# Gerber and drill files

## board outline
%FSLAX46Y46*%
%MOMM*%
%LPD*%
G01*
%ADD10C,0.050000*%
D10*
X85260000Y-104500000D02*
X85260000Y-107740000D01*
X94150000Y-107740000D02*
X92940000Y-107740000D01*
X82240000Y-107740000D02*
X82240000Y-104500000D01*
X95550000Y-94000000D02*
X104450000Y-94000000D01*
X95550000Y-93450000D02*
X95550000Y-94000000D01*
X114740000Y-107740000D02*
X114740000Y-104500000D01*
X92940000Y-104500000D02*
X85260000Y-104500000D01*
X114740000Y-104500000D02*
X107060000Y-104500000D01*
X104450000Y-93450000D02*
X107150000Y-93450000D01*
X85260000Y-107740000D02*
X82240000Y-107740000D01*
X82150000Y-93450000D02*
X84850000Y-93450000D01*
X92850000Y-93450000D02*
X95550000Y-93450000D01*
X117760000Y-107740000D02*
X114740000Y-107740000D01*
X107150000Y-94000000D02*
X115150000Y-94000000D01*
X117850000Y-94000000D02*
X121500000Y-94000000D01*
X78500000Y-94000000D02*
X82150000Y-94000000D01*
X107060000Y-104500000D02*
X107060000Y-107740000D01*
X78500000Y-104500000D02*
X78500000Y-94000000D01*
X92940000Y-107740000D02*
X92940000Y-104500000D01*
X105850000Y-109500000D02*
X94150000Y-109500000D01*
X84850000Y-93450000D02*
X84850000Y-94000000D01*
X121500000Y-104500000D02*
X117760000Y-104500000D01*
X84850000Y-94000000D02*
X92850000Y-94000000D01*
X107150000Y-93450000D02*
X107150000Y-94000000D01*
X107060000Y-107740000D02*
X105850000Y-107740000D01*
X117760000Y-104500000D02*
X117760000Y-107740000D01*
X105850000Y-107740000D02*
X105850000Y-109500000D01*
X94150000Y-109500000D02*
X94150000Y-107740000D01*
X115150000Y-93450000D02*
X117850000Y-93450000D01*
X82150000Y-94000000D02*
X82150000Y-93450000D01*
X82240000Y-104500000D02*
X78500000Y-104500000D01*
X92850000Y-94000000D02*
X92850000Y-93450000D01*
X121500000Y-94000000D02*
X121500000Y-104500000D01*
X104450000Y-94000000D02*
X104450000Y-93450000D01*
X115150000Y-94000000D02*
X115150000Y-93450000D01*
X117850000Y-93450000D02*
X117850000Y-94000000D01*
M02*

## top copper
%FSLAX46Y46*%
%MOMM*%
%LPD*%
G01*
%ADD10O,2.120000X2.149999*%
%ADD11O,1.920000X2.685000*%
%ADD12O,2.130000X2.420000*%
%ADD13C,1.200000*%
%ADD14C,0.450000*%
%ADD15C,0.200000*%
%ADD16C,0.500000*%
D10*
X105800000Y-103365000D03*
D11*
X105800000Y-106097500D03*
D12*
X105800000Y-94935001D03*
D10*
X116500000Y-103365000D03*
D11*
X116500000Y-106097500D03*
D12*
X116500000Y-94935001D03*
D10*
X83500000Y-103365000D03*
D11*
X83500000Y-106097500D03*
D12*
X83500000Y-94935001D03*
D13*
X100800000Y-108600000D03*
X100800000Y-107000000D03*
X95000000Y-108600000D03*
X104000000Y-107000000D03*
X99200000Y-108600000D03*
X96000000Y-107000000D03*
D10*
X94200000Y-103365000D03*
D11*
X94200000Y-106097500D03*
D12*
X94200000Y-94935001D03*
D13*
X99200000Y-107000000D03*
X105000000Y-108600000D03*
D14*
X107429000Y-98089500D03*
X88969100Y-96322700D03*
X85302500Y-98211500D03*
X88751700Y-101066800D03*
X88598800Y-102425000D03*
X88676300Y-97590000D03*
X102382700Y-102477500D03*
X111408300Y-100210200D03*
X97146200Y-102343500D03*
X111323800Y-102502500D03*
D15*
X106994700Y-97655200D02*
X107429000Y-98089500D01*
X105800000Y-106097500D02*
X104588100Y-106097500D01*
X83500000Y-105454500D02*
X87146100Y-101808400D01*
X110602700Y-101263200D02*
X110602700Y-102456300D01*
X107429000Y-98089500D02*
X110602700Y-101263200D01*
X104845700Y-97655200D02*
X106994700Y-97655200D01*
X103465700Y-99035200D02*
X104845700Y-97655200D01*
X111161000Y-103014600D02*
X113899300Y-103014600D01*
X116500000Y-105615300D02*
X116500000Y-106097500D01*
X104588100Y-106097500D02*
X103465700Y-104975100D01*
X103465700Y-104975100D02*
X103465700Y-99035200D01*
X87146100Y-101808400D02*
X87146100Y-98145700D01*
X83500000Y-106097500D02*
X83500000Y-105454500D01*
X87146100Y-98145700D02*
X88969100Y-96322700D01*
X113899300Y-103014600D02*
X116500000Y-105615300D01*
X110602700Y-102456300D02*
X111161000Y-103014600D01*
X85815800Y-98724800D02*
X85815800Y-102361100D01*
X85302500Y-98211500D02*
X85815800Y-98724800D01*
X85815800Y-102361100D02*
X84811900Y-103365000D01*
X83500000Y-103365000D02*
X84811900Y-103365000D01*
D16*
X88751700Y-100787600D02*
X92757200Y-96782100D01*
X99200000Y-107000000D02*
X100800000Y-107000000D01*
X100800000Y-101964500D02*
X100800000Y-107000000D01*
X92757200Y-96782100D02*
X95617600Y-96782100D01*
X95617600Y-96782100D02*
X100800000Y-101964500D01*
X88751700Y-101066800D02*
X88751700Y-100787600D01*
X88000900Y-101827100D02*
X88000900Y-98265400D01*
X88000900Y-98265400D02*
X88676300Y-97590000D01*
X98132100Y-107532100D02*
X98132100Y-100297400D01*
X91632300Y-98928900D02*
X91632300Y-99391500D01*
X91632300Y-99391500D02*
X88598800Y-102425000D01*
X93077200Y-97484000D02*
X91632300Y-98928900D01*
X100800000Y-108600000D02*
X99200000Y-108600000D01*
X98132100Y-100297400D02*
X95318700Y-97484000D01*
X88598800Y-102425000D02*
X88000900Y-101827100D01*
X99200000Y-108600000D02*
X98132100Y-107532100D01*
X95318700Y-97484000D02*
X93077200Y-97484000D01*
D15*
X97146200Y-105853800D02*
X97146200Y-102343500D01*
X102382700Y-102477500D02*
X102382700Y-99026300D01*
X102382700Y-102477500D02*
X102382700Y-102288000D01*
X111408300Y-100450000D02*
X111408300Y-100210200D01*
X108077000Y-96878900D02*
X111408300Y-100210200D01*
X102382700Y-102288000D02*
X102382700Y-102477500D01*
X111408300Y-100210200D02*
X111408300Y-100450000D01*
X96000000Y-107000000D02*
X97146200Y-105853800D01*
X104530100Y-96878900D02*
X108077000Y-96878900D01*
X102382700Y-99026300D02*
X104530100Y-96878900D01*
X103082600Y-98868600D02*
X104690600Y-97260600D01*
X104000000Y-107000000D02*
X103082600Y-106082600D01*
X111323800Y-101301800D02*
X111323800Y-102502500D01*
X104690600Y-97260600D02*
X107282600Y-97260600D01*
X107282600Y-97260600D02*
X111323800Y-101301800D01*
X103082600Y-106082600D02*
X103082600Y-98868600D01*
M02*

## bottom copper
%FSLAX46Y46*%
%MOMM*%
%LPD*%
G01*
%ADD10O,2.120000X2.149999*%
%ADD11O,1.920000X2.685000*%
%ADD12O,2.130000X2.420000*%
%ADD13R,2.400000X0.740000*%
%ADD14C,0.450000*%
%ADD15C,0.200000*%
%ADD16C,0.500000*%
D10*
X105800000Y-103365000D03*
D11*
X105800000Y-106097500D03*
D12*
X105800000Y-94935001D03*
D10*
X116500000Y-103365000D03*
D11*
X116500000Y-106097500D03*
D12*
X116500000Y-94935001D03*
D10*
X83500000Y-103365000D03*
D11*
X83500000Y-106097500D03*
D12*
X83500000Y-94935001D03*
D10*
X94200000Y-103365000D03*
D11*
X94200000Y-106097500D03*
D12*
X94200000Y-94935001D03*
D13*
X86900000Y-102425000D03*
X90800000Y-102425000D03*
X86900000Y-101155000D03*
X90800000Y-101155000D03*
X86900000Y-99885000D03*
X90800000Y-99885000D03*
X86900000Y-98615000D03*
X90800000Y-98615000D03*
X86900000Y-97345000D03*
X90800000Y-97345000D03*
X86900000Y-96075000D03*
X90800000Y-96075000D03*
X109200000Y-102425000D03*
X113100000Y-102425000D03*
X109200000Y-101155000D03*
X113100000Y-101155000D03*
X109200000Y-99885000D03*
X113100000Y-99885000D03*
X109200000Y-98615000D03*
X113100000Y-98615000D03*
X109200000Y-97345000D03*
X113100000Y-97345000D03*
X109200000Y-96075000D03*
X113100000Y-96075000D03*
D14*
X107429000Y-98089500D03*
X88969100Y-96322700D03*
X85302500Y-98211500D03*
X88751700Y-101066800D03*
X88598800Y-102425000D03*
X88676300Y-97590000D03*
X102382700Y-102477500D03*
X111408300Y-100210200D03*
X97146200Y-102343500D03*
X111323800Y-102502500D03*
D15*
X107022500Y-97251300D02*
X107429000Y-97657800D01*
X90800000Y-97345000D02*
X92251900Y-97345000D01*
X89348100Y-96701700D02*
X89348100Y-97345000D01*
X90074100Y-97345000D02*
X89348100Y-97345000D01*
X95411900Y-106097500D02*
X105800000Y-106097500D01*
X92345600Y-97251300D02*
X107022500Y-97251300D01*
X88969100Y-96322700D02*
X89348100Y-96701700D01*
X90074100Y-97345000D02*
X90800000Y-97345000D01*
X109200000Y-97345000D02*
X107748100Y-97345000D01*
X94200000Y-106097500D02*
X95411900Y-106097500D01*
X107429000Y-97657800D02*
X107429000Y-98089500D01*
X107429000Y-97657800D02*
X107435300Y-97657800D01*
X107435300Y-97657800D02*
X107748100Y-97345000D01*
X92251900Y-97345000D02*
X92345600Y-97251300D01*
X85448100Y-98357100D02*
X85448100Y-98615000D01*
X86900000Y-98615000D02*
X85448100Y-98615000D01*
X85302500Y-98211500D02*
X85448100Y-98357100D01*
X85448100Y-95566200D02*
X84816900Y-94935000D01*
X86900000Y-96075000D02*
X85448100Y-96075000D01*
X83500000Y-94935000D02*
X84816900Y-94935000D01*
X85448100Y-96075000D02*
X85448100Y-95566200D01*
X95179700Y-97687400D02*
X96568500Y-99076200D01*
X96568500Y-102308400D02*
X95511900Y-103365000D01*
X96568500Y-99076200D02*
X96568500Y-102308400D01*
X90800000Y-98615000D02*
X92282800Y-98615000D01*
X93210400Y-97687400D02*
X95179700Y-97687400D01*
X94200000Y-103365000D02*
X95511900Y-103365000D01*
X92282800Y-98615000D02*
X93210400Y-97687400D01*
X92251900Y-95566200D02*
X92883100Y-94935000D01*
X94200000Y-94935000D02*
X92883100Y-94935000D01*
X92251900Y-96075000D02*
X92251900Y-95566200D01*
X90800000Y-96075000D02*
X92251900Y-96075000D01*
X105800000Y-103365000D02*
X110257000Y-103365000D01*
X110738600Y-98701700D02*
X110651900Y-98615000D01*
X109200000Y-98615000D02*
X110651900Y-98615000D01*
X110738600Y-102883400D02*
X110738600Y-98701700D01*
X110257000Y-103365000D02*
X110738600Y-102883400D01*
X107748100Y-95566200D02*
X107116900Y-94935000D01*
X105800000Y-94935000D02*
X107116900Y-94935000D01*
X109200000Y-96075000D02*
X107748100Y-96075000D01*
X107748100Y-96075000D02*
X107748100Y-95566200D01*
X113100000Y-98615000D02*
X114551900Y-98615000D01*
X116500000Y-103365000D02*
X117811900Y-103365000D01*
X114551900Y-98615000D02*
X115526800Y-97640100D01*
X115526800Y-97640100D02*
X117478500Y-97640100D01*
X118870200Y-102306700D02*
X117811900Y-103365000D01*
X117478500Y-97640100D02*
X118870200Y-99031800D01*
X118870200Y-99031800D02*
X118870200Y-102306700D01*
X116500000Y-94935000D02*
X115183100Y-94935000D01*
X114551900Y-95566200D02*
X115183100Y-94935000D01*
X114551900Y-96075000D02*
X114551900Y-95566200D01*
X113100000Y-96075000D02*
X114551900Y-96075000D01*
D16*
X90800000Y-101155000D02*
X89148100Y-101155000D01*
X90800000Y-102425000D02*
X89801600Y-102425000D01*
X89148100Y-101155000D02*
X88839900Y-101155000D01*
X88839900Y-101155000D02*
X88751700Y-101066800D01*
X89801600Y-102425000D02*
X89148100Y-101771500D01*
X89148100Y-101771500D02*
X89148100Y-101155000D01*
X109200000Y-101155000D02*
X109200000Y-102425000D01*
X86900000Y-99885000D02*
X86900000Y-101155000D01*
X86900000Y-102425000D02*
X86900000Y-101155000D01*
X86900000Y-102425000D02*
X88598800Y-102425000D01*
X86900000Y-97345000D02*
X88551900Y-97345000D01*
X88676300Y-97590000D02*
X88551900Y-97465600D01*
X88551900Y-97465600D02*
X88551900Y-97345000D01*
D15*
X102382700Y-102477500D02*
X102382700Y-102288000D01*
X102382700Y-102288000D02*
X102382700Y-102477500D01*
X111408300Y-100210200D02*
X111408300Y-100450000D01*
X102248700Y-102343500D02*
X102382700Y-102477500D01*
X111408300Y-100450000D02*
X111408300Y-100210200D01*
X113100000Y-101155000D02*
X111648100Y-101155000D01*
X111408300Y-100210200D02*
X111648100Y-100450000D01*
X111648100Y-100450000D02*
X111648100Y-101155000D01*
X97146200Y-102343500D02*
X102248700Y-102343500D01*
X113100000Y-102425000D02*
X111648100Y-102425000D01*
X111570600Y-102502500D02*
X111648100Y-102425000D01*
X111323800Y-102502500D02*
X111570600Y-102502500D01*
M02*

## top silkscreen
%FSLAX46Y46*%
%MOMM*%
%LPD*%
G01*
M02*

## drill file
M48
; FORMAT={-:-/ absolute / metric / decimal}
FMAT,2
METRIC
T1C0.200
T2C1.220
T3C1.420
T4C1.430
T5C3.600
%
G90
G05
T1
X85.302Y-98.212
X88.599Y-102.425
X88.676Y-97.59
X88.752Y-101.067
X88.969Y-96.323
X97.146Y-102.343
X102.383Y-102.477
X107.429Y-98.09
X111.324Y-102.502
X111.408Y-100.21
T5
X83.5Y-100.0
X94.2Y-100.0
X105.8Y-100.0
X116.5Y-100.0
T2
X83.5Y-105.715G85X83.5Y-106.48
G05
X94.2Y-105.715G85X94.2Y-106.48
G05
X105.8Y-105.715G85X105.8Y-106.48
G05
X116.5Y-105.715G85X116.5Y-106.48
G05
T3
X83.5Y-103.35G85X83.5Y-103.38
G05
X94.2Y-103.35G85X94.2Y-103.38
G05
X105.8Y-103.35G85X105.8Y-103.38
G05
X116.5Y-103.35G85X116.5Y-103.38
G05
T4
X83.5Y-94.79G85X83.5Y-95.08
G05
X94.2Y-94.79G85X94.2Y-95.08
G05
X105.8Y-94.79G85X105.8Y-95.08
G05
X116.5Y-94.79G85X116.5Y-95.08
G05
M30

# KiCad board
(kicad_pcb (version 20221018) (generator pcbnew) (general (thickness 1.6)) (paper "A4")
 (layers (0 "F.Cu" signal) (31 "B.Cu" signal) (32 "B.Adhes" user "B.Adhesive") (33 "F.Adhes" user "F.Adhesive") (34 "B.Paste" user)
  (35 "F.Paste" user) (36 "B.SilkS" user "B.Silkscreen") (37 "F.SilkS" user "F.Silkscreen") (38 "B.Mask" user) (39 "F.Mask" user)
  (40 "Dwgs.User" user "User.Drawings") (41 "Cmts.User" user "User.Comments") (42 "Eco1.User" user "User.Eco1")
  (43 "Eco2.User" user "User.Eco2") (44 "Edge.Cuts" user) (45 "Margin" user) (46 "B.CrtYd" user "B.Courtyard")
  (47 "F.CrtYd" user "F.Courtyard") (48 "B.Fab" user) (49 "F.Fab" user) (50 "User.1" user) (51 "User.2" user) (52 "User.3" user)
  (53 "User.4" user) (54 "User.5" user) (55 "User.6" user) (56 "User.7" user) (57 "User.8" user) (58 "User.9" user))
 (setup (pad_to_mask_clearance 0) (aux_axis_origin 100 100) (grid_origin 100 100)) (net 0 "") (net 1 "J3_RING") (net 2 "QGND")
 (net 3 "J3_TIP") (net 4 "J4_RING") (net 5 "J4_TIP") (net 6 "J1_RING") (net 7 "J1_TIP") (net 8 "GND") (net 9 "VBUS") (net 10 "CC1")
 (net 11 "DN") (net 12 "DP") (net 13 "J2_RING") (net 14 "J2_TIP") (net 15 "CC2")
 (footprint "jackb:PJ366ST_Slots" (layer "F.Cu") (at 105.8 100)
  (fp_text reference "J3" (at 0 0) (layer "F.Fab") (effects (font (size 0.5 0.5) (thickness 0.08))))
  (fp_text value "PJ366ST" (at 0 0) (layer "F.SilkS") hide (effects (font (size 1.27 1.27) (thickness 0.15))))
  (pad "" np_thru_hole circle (at 0 0) (size 3.6 3.6) (drill 3.6) (layers "F&B.Cu" "*.Mask"))
  (pad "R" thru_hole oval (at 0 3.365) (size 2.12 2.149999) (drill oval 1.42 1.449999) (layers "*.Cu" "*.Mask") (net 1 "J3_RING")
   (thermal_bridge_angle 45))
  (pad "S" thru_hole oval (at 0 6.0975) (size 1.92 2.685) (drill oval 1.22 1.985) (layers "*.Cu" "*.Mask") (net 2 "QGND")
   (thermal_bridge_angle 45))
  (pad "T" thru_hole oval (at 0 -5.064999) (size 2.13 2.42) (drill oval 1.43 1.72) (layers "*.Cu" "*.Mask") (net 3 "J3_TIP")
   (thermal_bridge_angle 45)))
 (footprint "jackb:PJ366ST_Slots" (layer "F.Cu") (at 116.5 100)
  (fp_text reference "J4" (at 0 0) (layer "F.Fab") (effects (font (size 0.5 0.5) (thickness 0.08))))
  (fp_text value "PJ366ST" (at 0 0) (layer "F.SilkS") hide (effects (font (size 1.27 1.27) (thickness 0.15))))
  (pad "" np_thru_hole circle (at 0 0) (size 3.6 3.6) (drill 3.6) (layers "F&B.Cu" "*.Mask"))
  (pad "R" thru_hole oval (at 0 3.365) (size 2.12 2.149999) (drill oval 1.42 1.449999) (layers "*.Cu" "*.Mask") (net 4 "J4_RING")
   (thermal_bridge_angle 45))
  (pad "S" thru_hole oval (at 0 6.0975) (size 1.92 2.685) (drill oval 1.22 1.985) (layers "*.Cu" "*.Mask") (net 2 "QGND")
   (thermal_bridge_angle 45))
  (pad "T" thru_hole oval (at 0 -5.064999) (size 2.13 2.42) (drill oval 1.43 1.72) (layers "*.Cu" "*.Mask") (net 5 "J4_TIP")
   (thermal_bridge_angle 45)))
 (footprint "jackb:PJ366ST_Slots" (layer "F.Cu") (at 83.5 100)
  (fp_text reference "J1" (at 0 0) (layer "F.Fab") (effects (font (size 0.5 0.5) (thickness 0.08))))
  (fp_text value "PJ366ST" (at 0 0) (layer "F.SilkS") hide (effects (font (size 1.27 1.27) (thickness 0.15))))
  (pad "" np_thru_hole circle (at 0 0) (size 3.6 3.6) (drill 3.6) (layers "F&B.Cu" "*.Mask"))
  (pad "R" thru_hole oval (at 0 3.365) (size 2.12 2.149999) (drill oval 1.42 1.449999) (layers "*.Cu" "*.Mask") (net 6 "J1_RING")
   (thermal_bridge_angle 45))
  (pad "S" thru_hole oval (at 0 6.0975) (size 1.92 2.685) (drill oval 1.22 1.985) (layers "*.Cu" "*.Mask") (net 2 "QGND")
   (thermal_bridge_angle 45))
  (pad "T" thru_hole oval (at 0 -5.064999) (size 2.13 2.42) (drill oval 1.43 1.72) (layers "*.Cu" "*.Mask") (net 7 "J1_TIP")
   (thermal_bridge_angle 45)))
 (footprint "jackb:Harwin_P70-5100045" (layer "F.Cu") (at 100.8 108.6)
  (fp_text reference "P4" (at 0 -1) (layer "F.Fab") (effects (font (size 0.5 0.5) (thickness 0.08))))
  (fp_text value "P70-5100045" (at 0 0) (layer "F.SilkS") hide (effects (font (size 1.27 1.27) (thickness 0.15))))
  (pad "1" smd circle (at 0 0) (size 1.2 1.2) (layers "F.Cu" "F.Paste" "F.Mask") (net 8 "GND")))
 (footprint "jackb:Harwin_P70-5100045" (layer "F.Cu") (at 100.8 107)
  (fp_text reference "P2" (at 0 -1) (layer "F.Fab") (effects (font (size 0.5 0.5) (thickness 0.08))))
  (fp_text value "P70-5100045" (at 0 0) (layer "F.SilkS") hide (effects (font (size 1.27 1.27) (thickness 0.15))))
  (pad "1" smd circle (at 0 0) (size 1.2 1.2) (layers "F.Cu" "F.Paste" "F.Mask") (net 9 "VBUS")))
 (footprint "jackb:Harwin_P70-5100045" (layer "F.Cu") (at 95 108.6)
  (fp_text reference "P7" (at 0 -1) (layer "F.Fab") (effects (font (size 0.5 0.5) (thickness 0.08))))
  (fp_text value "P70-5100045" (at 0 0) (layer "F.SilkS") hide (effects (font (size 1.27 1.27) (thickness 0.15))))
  (pad "1" smd circle (at 0 0) (size 1.2 1.2) (layers "F.Cu" "F.Paste" "F.Mask") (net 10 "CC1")))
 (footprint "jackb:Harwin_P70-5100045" (layer "F.Cu") (at 104 107)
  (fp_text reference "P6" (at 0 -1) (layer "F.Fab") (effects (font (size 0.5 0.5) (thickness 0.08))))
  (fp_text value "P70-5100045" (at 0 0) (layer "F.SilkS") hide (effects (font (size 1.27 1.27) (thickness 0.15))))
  (pad "1" smd circle (at 0 0) (size 1.2 1.2) (layers "F.Cu" "F.Paste" "F.Mask") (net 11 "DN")))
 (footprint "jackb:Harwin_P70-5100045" (layer "F.Cu") (at 99.2 108.6)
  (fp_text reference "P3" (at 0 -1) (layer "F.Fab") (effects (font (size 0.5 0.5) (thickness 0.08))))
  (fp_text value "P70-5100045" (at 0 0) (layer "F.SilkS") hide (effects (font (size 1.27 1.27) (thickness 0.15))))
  (pad "1" smd circle (at 0 0) (size 1.2 1.2) (layers "F.Cu" "F.Paste" "F.Mask") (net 8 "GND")))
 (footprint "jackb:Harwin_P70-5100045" (layer "F.Cu") (at 96 107)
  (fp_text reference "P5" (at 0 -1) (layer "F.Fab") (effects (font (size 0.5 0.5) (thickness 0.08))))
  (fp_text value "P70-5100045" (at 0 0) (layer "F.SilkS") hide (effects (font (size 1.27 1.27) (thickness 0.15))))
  (pad "1" smd circle (at 0 0) (size 1.2 1.2) (layers "F.Cu" "F.Paste" "F.Mask") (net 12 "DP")))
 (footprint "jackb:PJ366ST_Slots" (layer "F.Cu") (at 94.2 100)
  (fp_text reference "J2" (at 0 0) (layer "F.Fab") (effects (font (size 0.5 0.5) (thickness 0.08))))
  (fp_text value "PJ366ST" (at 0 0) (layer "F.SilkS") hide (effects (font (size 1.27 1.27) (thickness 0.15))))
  (pad "" np_thru_hole circle (at 0 0) (size 3.6 3.6) (drill 3.6) (layers "F&B.Cu" "*.Mask"))
  (pad "R" thru_hole oval (at 0 3.365) (size 2.12 2.149999) (drill oval 1.42 1.449999) (layers "*.Cu" "*.Mask") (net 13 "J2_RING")
   (thermal_bridge_angle 45))
  (pad "S" thru_hole oval (at 0 6.0975) (size 1.92 2.685) (drill oval 1.22 1.985) (layers "*.Cu" "*.Mask") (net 2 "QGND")
   (thermal_bridge_angle 45))
  (pad "T" thru_hole oval (at 0 -5.064999) (size 2.13 2.42) (drill oval 1.43 1.72) (layers "*.Cu" "*.Mask") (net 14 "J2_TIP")
   (thermal_bridge_angle 45)))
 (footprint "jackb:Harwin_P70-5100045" (layer "F.Cu") (at 99.2 107)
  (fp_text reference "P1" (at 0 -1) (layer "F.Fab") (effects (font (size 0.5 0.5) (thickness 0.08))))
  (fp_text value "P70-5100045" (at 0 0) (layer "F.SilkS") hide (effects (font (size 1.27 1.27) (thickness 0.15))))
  (pad "1" smd circle (at 0 0) (size 1.2 1.2) (layers "F.Cu" "F.Paste" "F.Mask") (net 9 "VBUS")))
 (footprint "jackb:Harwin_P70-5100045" (layer "F.Cu") (at 105 108.6)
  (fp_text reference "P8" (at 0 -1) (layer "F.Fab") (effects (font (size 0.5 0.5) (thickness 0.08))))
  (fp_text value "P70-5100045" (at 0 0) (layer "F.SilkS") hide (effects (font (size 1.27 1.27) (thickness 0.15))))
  (pad "1" smd circle (at 0 0) (size 1.2 1.2) (layers "F.Cu" "F.Paste" "F.Mask") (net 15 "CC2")))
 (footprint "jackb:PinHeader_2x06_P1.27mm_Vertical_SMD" (layer "B.Cu") (at 88.85 99.25)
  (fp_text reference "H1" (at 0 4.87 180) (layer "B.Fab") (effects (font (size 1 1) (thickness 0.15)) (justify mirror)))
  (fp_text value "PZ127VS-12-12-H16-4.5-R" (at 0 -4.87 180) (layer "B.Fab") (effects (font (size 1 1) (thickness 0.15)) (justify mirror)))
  (pad "1" smd rect (at -1.95 3.175) (size 2.4 0.74) (layers "B.Cu" "B.Paste" "B.Mask") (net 8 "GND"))
  (pad "2" smd rect (at 1.95 3.175) (size 2.4 0.74) (layers "B.Cu" "B.Paste" "B.Mask") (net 9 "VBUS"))
  (pad "3" smd rect (at -1.95 1.905) (size 2.4 0.74) (layers "B.Cu" "B.Paste" "B.Mask") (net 8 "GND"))
  (pad "4" smd rect (at 1.95 1.905) (size 2.4 0.74) (layers "B.Cu" "B.Paste" "B.Mask") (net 9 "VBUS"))
  (pad "5" smd rect (at -1.95 0.635) (size 2.4 0.74) (layers "B.Cu" "B.Paste" "B.Mask") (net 8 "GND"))
  (pad "6" smd rect (at 1.95 0.635) (size 2.4 0.74) (layers "B.Cu" "B.Paste" "B.Mask") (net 10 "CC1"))
  (pad "7" smd rect (at -1.95 -0.635) (size 2.4 0.74) (layers "B.Cu" "B.Paste" "B.Mask") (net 6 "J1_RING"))
  (pad "8" smd rect (at 1.95 -0.635) (size 2.4 0.74) (layers "B.Cu" "B.Paste" "B.Mask") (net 13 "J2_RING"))
  (pad "9" smd rect (at -1.95 -1.905) (size 2.4 0.74) (layers "B.Cu" "B.Paste" "B.Mask") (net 8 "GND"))
  (pad "10" smd rect (at 1.95 -1.905) (size 2.4 0.74) (layers "B.Cu" "B.Paste" "B.Mask") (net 2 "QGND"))
  (pad "11" smd rect (at -1.95 -3.175) (size 2.4 0.74) (layers "B.Cu" "B.Paste" "B.Mask") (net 7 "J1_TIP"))
  (pad "12" smd rect (at 1.95 -3.175) (size 2.4 0.74) (layers "B.Cu" "B.Paste" "B.Mask") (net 14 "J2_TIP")))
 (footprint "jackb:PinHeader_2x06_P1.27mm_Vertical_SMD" (layer "B.Cu") (at 111.15 99.25)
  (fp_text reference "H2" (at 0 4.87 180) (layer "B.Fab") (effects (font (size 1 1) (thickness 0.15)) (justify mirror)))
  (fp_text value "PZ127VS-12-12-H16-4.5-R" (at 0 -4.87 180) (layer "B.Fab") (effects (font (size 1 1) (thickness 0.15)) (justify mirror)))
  (pad "1" smd rect (at -1.95 3.175) (size 2.4 0.74) (layers "B.Cu" "B.Paste" "B.Mask") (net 9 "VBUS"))
  (pad "2" smd rect (at 1.95 3.175) (size 2.4 0.74) (layers "B.Cu" "B.Paste" "B.Mask") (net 11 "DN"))
  (pad "3" smd rect (at -1.95 1.905) (size 2.4 0.74) (layers "B.Cu" "B.Paste" "B.Mask") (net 9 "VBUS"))
  (pad "4" smd rect (at 1.95 1.905) (size 2.4 0.74) (layers "B.Cu" "B.Paste" "B.Mask") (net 12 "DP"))
  (pad "5" smd rect (at -1.95 0.635) (size 2.4 0.74) (layers "B.Cu" "B.Paste" "B.Mask") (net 15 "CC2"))
  (pad "6" smd rect (at 1.95 0.635) (size 2.4 0.74) (layers "B.Cu" "B.Paste" "B.Mask") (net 8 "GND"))
  (pad "7" smd rect (at -1.95 -0.635) (size 2.4 0.74) (layers "B.Cu" "B.Paste" "B.Mask") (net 1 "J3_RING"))
  (pad "8" smd rect (at 1.95 -0.635) (size 2.4 0.74) (layers "B.Cu" "B.Paste" "B.Mask") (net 4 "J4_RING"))
  (pad "9" smd rect (at -1.95 -1.905) (size 2.4 0.74) (layers "B.Cu" "B.Paste" "B.Mask") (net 2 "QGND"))
  (pad "10" smd rect (at 1.95 -1.905) (size 2.4 0.74) (layers "B.Cu" "B.Paste" "B.Mask") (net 8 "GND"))
  (pad "11" smd rect (at -1.95 -3.175) (size 2.4 0.74) (layers "B.Cu" "B.Paste" "B.Mask") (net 3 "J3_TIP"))
  (pad "12" smd rect (at 1.95 -3.175) (size 2.4 0.74) (layers "B.Cu" "B.Paste" "B.Mask") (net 5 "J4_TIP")))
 (gr_line (start 85.26 104.5) (end 85.26 107.74) (stroke (width 0.05) (type default)) (layer "Edge.Cuts"))
 (gr_line (start 94.15 107.74) (end 92.94 107.74) (stroke (width 0.05) (type default)) (layer "Edge.Cuts"))
 (gr_line (start 82.24 107.74) (end 82.24 104.5) (stroke (width 0.05) (type default)) (layer "Edge.Cuts"))
 (gr_line (start 95.55 94) (end 104.45 94) (stroke (width 0.05) (type default)) (layer "Edge.Cuts"))
 (gr_line (start 95.55 93.45) (end 95.55 94) (stroke (width 0.05) (type default)) (layer "Edge.Cuts"))
 (gr_line (start 114.74 107.74) (end 114.74 104.5) (stroke (width 0.05) (type default)) (layer "Edge.Cuts"))
 (gr_line (start 92.94 104.5) (end 85.26 104.5) (stroke (width 0.05) (type default)) (layer "Edge.Cuts"))
 (gr_line (start 114.74 104.5) (end 107.06 104.5) (stroke (width 0.05) (type default)) (layer "Edge.Cuts"))
 (gr_line (start 104.45 93.45) (end 107.15 93.45) (stroke (width 0.05) (type default)) (layer "Edge.Cuts"))
 (gr_line (start 85.26 107.74) (end 82.24 107.74) (stroke (width 0.05) (type default)) (layer "Edge.Cuts"))
 (gr_line (start 82.15 93.45) (end 84.85 93.45) (stroke (width 0.05) (type default)) (layer "Edge.Cuts"))
 (gr_line (start 92.85 93.45) (end 95.55 93.45) (stroke (width 0.05) (type default)) (layer "Edge.Cuts"))
 (gr_line (start 117.76 107.74) (end 114.74 107.74) (stroke (width 0.05) (type default)) (layer "Edge.Cuts"))
 (gr_line (start 107.15 94) (end 115.15 94) (stroke (width 0.05) (type default)) (layer "Edge.Cuts"))
 (gr_line (start 117.85 94) (end 121.5 94) (stroke (width 0.05) (type default)) (layer "Edge.Cuts"))
 (gr_line (start 78.5 94) (end 82.15 94) (stroke (width 0.05) (type default)) (layer "Edge.Cuts"))
 (gr_line (start 107.06 104.5) (end 107.06 107.74) (stroke (width 0.05) (type default)) (layer "Edge.Cuts"))
 (gr_line (start 78.5 104.5) (end 78.5 94) (stroke (width 0.05) (type default)) (layer "Edge.Cuts"))
 (gr_line (start 92.94 107.74) (end 92.94 104.5) (stroke (width 0.05) (type default)) (layer "Edge.Cuts"))
 (gr_line (start 105.85 109.5) (end 94.15 109.5) (stroke (width 0.05) (type default)) (layer "Edge.Cuts"))
 (gr_line (start 84.85 93.45) (end 84.85 94) (stroke (width 0.05) (type default)) (layer "Edge.Cuts"))
 (gr_line (start 121.5 104.5) (end 117.76 104.5) (stroke (width 0.05) (type default)) (layer "Edge.Cuts"))
 (gr_line (start 84.85 94) (end 92.85 94) (stroke (width 0.05) (type default)) (layer "Edge.Cuts"))
 (gr_line (start 107.15 93.45) (end 107.15 94) (stroke (width 0.05) (type default)) (layer "Edge.Cuts"))
 (gr_line (start 107.06 107.74) (end 105.85 107.74) (stroke (width 0.05) (type default)) (layer "Edge.Cuts"))
 (gr_line (start 117.76 104.5) (end 117.76 107.74) (stroke (width 0.05) (type default)) (layer "Edge.Cuts"))
 (gr_line (start 105.85 107.74) (end 105.85 109.5) (stroke (width 0.05) (type default)) (layer "Edge.Cuts"))
 (gr_line (start 94.15 109.5) (end 94.15 107.74) (stroke (width 0.05) (type default)) (layer "Edge.Cuts"))
 (gr_line (start 115.15 93.45) (end 117.85 93.45) (stroke (width 0.05) (type default)) (layer "Edge.Cuts"))
 (gr_line (start 82.15 94) (end 82.15 93.45) (stroke (width 0.05) (type default)) (layer "Edge.Cuts"))
 (gr_line (start 82.24 104.5) (end 78.5 104.5) (stroke (width 0.05) (type default)) (layer "Edge.Cuts"))
 (gr_line (start 92.85 94) (end 92.85 93.45) (stroke (width 0.05) (type default)) (layer "Edge.Cuts"))
 (gr_line (start 121.5 94) (end 121.5 104.5) (stroke (width 0.05) (type default)) (layer "Edge.Cuts"))
 (gr_line (start 104.45 94) (end 104.45 93.45) (stroke (width 0.05) (type default)) (layer "Edge.Cuts"))
 (gr_line (start 115.15 94) (end 115.15 93.45) (stroke (width 0.05) (type default)) (layer "Edge.Cuts"))
 (gr_line (start 117.85 93.45) (end 117.85 94) (stroke (width 0.05) (type default)) (layer "Edge.Cuts"))
 (segment (start 106.9947 97.6552) (end 107.429 98.0895) (width 0.2) (layer "F.Cu") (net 2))
 (segment (start 105.8 106.0975) (end 104.5881 106.0975) (width 0.2) (layer "F.Cu") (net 2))
 (segment (start 83.5 105.4545) (end 87.1461 101.8084) (width 0.2) (layer "F.Cu") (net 2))
 (segment (start 110.6027 101.2632) (end 110.6027 102.4563) (width 0.2) (layer "F.Cu") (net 2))
 (segment (start 107.429 98.0895) (end 110.6027 101.2632) (width 0.2) (layer "F.Cu") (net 2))
 (segment (start 104.8457 97.6552) (end 106.9947 97.6552) (width 0.2) (layer "F.Cu") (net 2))
 (segment (start 103.4657 99.0352) (end 104.8457 97.6552) (width 0.2) (layer "F.Cu") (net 2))
 (segment (start 111.161 103.0146) (end 113.8993 103.0146) (width 0.2) (layer "F.Cu") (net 2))
 (segment (start 116.5 105.6153) (end 116.5 106.0975) (width 0.2) (layer "F.Cu") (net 2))
 (segment (start 104.5881 106.0975) (end 103.4657 104.9751) (width 0.2) (layer "F.Cu") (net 2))
 (segment (start 103.4657 104.9751) (end 103.4657 99.0352) (width 0.2) (layer "F.Cu") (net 2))
 (segment (start 87.1461 101.8084) (end 87.1461 98.1457) (width 0.2) (layer "F.Cu") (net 2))
 (segment (start 83.5 106.0975) (end 83.5 105.4545) (width 0.2) (layer "F.Cu") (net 2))
 (segment (start 87.1461 98.1457) (end 88.9691 96.3227) (width 0.2) (layer "F.Cu") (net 2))
 (segment (start 113.8993 103.0146) (end 116.5 105.6153) (width 0.2) (layer "F.Cu") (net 2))
 (segment (start 110.6027 102.4563) (end 111.161 103.0146) (width 0.2) (layer "F.Cu") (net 2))
 (via (at 107.429 98.0895) (size 0.45) (drill 0.2) (layers "F.Cu" "B.Cu") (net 2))
 (via (at 88.9691 96.3227) (size 0.45) (drill 0.2) (layers "F.Cu" "B.Cu") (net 2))
 (segment (start 107.0225 97.2513) (end 107.429 97.6578) (width 0.2) (layer "B.Cu") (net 2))
 (segment (start 90.8 97.345) (end 92.2519 97.345) (width 0.2) (layer "B.Cu") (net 2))
 (segment (start 89.3481 96.7017) (end 89.3481 97.345) (width 0.2) (layer "B.Cu") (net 2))
 (segment (start 90.0741 97.345) (end 89.3481 97.345) (width 0.2) (layer "B.Cu") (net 2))
 (segment (start 95.4119 106.0975) (end 105.8 106.0975) (width 0.2) (layer "B.Cu") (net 2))
 (segment (start 92.3456 97.2513) (end 107.0225 97.2513) (width 0.2) (layer "B.Cu") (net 2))
 (segment (start 88.9691 96.3227) (end 89.3481 96.7017) (width 0.2) (layer "B.Cu") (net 2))
 (segment (start 90.0741 97.345) (end 90.8 97.345) (width 0.2) (layer "B.Cu") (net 2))
 (segment (start 109.2 97.345) (end 107.7481 97.345) (width 0.2) (layer "B.Cu") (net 2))
 (segment (start 94.2 106.0975) (end 95.4119 106.0975) (width 0.2) (layer "B.Cu") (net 2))
 (segment (start 107.429 97.6578) (end 107.429 98.0895) (width 0.2) (layer "B.Cu") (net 2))
 (segment (start 107.429 97.6578) (end 107.4353 97.6578) (width 0.2) (layer "B.Cu") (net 2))
 (segment (start 107.4353 97.6578) (end 107.7481 97.345) (width 0.2) (layer "B.Cu") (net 2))
 (segment (start 92.2519 97.345) (end 92.3456 97.2513) (width 0.2) (layer "B.Cu") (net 2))
 (segment (start 85.8158 98.7248) (end 85.8158 102.3611) (width 0.2) (layer "F.Cu") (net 6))
 (segment (start 85.3025 98.2115) (end 85.8158 98.7248) (width 0.2) (layer "F.Cu") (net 6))
 (segment (start 85.8158 102.3611) (end 84.8119 103.365) (width 0.2) (layer "F.Cu") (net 6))
 (segment (start 83.5 103.365) (end 84.8119 103.365) (width 0.2) (layer "F.Cu") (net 6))
 (via (at 85.3025 98.2115) (size 0.45) (drill 0.2) (layers "F.Cu" "B.Cu") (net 6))
 (segment (start 85.4481 98.3571) (end 85.4481 98.615) (width 0.2) (layer "B.Cu") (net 6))
 (segment (start 86.9 98.615) (end 85.4481 98.615) (width 0.2) (layer "B.Cu") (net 6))
 (segment (start 85.3025 98.2115) (end 85.4481 98.3571) (width 0.2) (layer "B.Cu") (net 6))
 (segment (start 85.4481 95.5662) (end 84.8169 94.935) (width 0.2) (layer "B.Cu") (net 7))
 (segment (start 86.9 96.075) (end 85.4481 96.075) (width 0.2) (layer "B.Cu") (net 7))
 (segment (start 83.5 94.935) (end 84.8169 94.935) (width 0.2) (layer "B.Cu") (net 7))
 (segment (start 85.4481 96.075) (end 85.4481 95.5662) (width 0.2) (layer "B.Cu") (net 7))
 (segment (start 95.1797 97.6874) (end 96.5685 99.0762) (width 0.2) (layer "B.Cu") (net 13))
 (segment (start 96.5685 102.3084) (end 95.5119 103.365) (width 0.2) (layer "B.Cu") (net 13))
 (segment (start 96.5685 99.0762) (end 96.5685 102.3084) (width 0.2) (layer "B.Cu") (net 13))
 (segment (start 90.8 98.615) (end 92.2828 98.615) (width 0.2) (layer "B.Cu") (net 13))
 (segment (start 93.2104 97.6874) (end 95.1797 97.6874) (width 0.2) (layer "B.Cu") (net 13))
 (segment (start 94.2 103.365) (end 95.5119 103.365) (width 0.2) (layer "B.Cu") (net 13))
 (segment (start 92.2828 98.615) (end 93.2104 97.6874) (width 0.2) (layer "B.Cu") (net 13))
 (segment (start 92.2519 95.5662) (end 92.8831 94.935) (width 0.2) (layer "B.Cu") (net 14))
 (segment (start 94.2 94.935) (end 92.8831 94.935) (width 0.2) (layer "B.Cu") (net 14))
 (segment (start 92.2519 96.075) (end 92.2519 95.5662) (width 0.2) (layer "B.Cu") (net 14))
 (segment (start 90.8 96.075) (end 92.2519 96.075) (width 0.2) (layer "B.Cu") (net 14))
 (segment (start 105.8 103.365) (end 110.257 103.365) (width 0.2) (layer "B.Cu") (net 1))
 (segment (start 110.7386 98.7017) (end 110.6519 98.615) (width 0.2) (layer "B.Cu") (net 1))
 (segment (start 109.2 98.615) (end 110.6519 98.615) (width 0.2) (layer "B.Cu") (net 1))
 (segment (start 110.7386 102.8834) (end 110.7386 98.7017) (width 0.2) (layer "B.Cu") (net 1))
 (segment (start 110.257 103.365) (end 110.7386 102.8834) (width 0.2) (layer "B.Cu") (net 1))
 (segment (start 107.7481 95.5662) (end 107.1169 94.935) (width 0.2) (layer "B.Cu") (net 3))
 (segment (start 105.8 94.935) (end 107.1169 94.935) (width 0.2) (layer "B.Cu") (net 3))
 (segment (start 109.2 96.075) (end 107.7481 96.075) (width 0.2) (layer "B.Cu") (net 3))
 (segment (start 107.7481 96.075) (end 107.7481 95.5662) (width 0.2) (layer "B.Cu") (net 3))
 (segment (start 113.1 98.615) (end 114.5519 98.615) (width 0.2) (layer "B.Cu") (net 4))
 (segment (start 116.5 103.365) (end 117.8119 103.365) (width 0.2) (layer "B.Cu") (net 4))
 (segment (start 114.5519 98.615) (end 115.5268 97.6401) (width 0.2) (layer "B.Cu") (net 4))
 (segment (start 115.5268 97.6401) (end 117.4785 97.6401) (width 0.2) (layer "B.Cu") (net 4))
 (segment (start 118.8702 102.3067) (end 117.8119 103.365) (width 0.2) (layer "B.Cu") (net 4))
 (segment (start 117.4785 97.6401) (end 118.8702 99.0318) (width 0.2) (layer "B.Cu") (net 4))
 (segment (start 118.8702 99.0318) (end 118.8702 102.3067) (width 0.2) (layer "B.Cu") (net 4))
 (segment (start 116.5 94.935) (end 115.1831 94.935) (width 0.2) (layer "B.Cu") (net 5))
 (segment (start 114.5519 95.5662) (end 115.1831 94.935) (width 0.2) (layer "B.Cu") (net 5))
 (segment (start 114.5519 96.075) (end 114.5519 95.5662) (width 0.2) (layer "B.Cu") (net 5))
 (segment (start 113.1 96.075) (end 114.5519 96.075) (width 0.2) (layer "B.Cu") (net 5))
 (segment (start 88.7517 100.7876) (end 92.7572 96.7821) (width 0.5) (layer "F.Cu") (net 9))
 (segment (start 99.2 107) (end 100.8 107) (width 0.5) (layer "F.Cu") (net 9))
 (segment (start 100.8 101.9645) (end 100.8 107) (width 0.5) (layer "F.Cu") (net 9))
 (segment (start 92.7572 96.7821) (end 95.6176 96.7821) (width 0.5) (layer "F.Cu") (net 9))
 (segment (start 95.6176 96.7821) (end 100.8 101.9645) (width 0.5) (layer "F.Cu") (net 9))
 (segment (start 88.7517 101.0668) (end 88.7517 100.7876) (width 0.5) (layer "F.Cu") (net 9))
 (via (at 88.7517 101.0668) (size 0.45) (drill 0.2) (layers "F.Cu" "B.Cu") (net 9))
 (segment (start 90.8 101.155) (end 89.1481 101.155) (width 0.5) (layer "B.Cu") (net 9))
 (segment (start 90.8 102.425) (end 89.8016 102.425) (width 0.5) (layer "B.Cu") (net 9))
 (segment (start 89.1481 101.155) (end 88.8399 101.155) (width 0.5) (layer "B.Cu") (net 9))
 (segment (start 88.8399 101.155) (end 88.7517 101.0668) (width 0.5) (layer "B.Cu") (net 9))
 (segment (start 89.8016 102.425) (end 89.1481 101.7715) (width 0.5) (layer "B.Cu") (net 9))
 (segment (start 89.1481 101.7715) (end 89.1481 101.155) (width 0.5) (layer "B.Cu") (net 9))
 (segment (start 109.2 101.155) (end 109.2 102.425) (width 0.5) (layer "B.Cu") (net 9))
 (segment (start 88.0009 101.8271) (end 88.0009 98.2654) (width 0.5) (layer "F.Cu") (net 8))
 (segment (start 88.0009 98.2654) (end 88.6763 97.59) (width 0.5) (layer "F.Cu") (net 8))
 (segment (start 98.1321 107.5321) (end 98.1321 100.2974) (width 0.5) (layer "F.Cu") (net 8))
 (segment (start 91.6323 98.9289) (end 91.6323 99.3915) (width 0.5) (layer "F.Cu") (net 8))
 (segment (start 91.6323 99.3915) (end 88.5988 102.425) (width 0.5) (layer "F.Cu") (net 8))
 (segment (start 93.0772 97.484) (end 91.6323 98.9289) (width 0.5) (layer "F.Cu") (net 8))
 (segment (start 100.8 108.6) (end 99.2 108.6) (width 0.5) (layer "F.Cu") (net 8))
 (segment (start 98.1321 100.2974) (end 95.3187 97.484) (width 0.5) (layer "F.Cu") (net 8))
 (segment (start 88.5988 102.425) (end 88.0009 101.8271) (width 0.5) (layer "F.Cu") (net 8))
 (segment (start 99.2 108.6) (end 98.1321 107.5321) (width 0.5) (layer "F.Cu") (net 8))
 (segment (start 95.3187 97.484) (end 93.0772 97.484) (width 0.5) (layer "F.Cu") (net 8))
 (via (at 88.5988 102.425) (size 0.45) (drill 0.2) (layers "F.Cu" "B.Cu") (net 8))
 (via (at 88.6763 97.59) (size 0.45) (drill 0.2) (layers "F.Cu" "B.Cu") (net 8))
 (segment (start 86.9 99.885) (end 86.9 101.155) (width 0.5) (layer "B.Cu") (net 8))
 (segment (start 86.9 102.425) (end 86.9 101.155) (width 0.5) (layer "B.Cu") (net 8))
 (segment (start 86.9 102.425) (end 88.5988 102.425) (width 0.5) (layer "B.Cu") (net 8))
 (segment (start 86.9 97.345) (end 88.5519 97.345) (width 0.5) (layer "B.Cu") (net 8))
 (segment (start 88.6763 97.59) (end 88.5519 97.4656) (width 0.5) (layer "B.Cu") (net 8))
 (segment (start 88.5519 97.4656) (end 88.5519 97.345) (width 0.5) (layer "B.Cu") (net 8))
 (segment (start 97.1462 105.8538) (end 97.1462 102.3435) (width 0.2) (layer "F.Cu") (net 12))
 (segment (start 102.3827 102.4775) (end 102.3827 99.0263) (width 0.2) (layer "F.Cu") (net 12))
 (segment (start 102.3827 102.4775) (end 102.3827 102.288) (width 0.2) (layer "F.Cu") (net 12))
 (segment (start 111.4083 100.45) (end 111.4083 100.2102) (width 0.2) (layer "F.Cu") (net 12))
 (segment (start 108.077 96.8789) (end 111.4083 100.2102) (width 0.2) (layer "F.Cu") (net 12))
 (segment (start 102.3827 102.288) (end 102.3827 102.4775) (width 0.2) (layer "F.Cu") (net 12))
 (segment (start 111.4083 100.2102) (end 111.4083 100.45) (width 0.2) (layer "F.Cu") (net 12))
 (segment (start 96 107) (end 97.1462 105.8538) (width 0.2) (layer "F.Cu") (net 12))
 (segment (start 104.5301 96.8789) (end 108.077 96.8789) (width 0.2) (layer "F.Cu") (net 12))
 (segment (start 102.3827 99.0263) (end 104.5301 96.8789) (width 0.2) (layer "F.Cu") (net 12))
 (via (at 102.3827 102.4775) (size 0.45) (drill 0.2) (layers "F.Cu" "B.Cu") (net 12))
 (via (at 111.4083 100.2102) (size 0.45) (drill 0.2) (layers "F.Cu" "B.Cu") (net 12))
 (via (at 97.1462 102.3435) (size 0.45) (drill 0.2) (layers "F.Cu" "B.Cu") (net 12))
 (segment (start 102.3827 102.4775) (end 102.3827 102.288) (width 0.2) (layer "B.Cu") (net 12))
 (segment (start 102.3827 102.288) (end 102.3827 102.4775) (width 0.2) (layer "B.Cu") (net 12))
 (segment (start 111.4083 100.2102) (end 111.4083 100.45) (width 0.2) (layer "B.Cu") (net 12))
 (segment (start 102.2487 102.3435) (end 102.3827 102.4775) (width 0.2) (layer "B.Cu") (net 12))
 (segment (start 111.4083 100.45) (end 111.4083 100.2102) (width 0.2) (layer "B.Cu") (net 12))
 (segment (start 113.1 101.155) (end 111.6481 101.155) (width 0.2) (layer "B.Cu") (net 12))
 (segment (start 111.4083 100.2102) (end 111.6481 100.45) (width 0.2) (layer "B.Cu") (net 12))
 (segment (start 111.6481 100.45) (end 111.6481 101.155) (width 0.2) (layer "B.Cu") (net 12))
 (segment (start 97.1462 102.3435) (end 102.2487 102.3435) (width 0.2) (layer "B.Cu") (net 12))
 (segment (start 103.0826 98.8686) (end 104.6906 97.2606) (width 0.2) (layer "F.Cu") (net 11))
 (segment (start 104 107) (end 103.0826 106.0826) (width 0.2) (layer "F.Cu") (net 11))
 (segment (start 111.3238 101.3018) (end 111.3238 102.5025) (width 0.2) (layer "F.Cu") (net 11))
 (segment (start 104.6906 97.2606) (end 107.2826 97.2606) (width 0.2) (layer "F.Cu") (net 11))
 (segment (start 107.2826 97.2606) (end 111.3238 101.3018) (width 0.2) (layer "F.Cu") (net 11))
 (segment (start 103.0826 106.0826) (end 103.0826 98.8686) (width 0.2) (layer "F.Cu") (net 11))
 (via (at 111.3238 102.5025) (size 0.45) (drill 0.2) (layers "F.Cu" "B.Cu") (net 11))
 (segment (start 113.1 102.425) (end 111.6481 102.425) (width 0.2) (layer "B.Cu") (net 11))
 (segment (start 111.5706 102.5025) (end 111.6481 102.425) (width 0.2) (layer "B.Cu") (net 11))
 (segment (start 111.3238 102.5025) (end 111.5706 102.5025) (width 0.2) (layer "B.Cu") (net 11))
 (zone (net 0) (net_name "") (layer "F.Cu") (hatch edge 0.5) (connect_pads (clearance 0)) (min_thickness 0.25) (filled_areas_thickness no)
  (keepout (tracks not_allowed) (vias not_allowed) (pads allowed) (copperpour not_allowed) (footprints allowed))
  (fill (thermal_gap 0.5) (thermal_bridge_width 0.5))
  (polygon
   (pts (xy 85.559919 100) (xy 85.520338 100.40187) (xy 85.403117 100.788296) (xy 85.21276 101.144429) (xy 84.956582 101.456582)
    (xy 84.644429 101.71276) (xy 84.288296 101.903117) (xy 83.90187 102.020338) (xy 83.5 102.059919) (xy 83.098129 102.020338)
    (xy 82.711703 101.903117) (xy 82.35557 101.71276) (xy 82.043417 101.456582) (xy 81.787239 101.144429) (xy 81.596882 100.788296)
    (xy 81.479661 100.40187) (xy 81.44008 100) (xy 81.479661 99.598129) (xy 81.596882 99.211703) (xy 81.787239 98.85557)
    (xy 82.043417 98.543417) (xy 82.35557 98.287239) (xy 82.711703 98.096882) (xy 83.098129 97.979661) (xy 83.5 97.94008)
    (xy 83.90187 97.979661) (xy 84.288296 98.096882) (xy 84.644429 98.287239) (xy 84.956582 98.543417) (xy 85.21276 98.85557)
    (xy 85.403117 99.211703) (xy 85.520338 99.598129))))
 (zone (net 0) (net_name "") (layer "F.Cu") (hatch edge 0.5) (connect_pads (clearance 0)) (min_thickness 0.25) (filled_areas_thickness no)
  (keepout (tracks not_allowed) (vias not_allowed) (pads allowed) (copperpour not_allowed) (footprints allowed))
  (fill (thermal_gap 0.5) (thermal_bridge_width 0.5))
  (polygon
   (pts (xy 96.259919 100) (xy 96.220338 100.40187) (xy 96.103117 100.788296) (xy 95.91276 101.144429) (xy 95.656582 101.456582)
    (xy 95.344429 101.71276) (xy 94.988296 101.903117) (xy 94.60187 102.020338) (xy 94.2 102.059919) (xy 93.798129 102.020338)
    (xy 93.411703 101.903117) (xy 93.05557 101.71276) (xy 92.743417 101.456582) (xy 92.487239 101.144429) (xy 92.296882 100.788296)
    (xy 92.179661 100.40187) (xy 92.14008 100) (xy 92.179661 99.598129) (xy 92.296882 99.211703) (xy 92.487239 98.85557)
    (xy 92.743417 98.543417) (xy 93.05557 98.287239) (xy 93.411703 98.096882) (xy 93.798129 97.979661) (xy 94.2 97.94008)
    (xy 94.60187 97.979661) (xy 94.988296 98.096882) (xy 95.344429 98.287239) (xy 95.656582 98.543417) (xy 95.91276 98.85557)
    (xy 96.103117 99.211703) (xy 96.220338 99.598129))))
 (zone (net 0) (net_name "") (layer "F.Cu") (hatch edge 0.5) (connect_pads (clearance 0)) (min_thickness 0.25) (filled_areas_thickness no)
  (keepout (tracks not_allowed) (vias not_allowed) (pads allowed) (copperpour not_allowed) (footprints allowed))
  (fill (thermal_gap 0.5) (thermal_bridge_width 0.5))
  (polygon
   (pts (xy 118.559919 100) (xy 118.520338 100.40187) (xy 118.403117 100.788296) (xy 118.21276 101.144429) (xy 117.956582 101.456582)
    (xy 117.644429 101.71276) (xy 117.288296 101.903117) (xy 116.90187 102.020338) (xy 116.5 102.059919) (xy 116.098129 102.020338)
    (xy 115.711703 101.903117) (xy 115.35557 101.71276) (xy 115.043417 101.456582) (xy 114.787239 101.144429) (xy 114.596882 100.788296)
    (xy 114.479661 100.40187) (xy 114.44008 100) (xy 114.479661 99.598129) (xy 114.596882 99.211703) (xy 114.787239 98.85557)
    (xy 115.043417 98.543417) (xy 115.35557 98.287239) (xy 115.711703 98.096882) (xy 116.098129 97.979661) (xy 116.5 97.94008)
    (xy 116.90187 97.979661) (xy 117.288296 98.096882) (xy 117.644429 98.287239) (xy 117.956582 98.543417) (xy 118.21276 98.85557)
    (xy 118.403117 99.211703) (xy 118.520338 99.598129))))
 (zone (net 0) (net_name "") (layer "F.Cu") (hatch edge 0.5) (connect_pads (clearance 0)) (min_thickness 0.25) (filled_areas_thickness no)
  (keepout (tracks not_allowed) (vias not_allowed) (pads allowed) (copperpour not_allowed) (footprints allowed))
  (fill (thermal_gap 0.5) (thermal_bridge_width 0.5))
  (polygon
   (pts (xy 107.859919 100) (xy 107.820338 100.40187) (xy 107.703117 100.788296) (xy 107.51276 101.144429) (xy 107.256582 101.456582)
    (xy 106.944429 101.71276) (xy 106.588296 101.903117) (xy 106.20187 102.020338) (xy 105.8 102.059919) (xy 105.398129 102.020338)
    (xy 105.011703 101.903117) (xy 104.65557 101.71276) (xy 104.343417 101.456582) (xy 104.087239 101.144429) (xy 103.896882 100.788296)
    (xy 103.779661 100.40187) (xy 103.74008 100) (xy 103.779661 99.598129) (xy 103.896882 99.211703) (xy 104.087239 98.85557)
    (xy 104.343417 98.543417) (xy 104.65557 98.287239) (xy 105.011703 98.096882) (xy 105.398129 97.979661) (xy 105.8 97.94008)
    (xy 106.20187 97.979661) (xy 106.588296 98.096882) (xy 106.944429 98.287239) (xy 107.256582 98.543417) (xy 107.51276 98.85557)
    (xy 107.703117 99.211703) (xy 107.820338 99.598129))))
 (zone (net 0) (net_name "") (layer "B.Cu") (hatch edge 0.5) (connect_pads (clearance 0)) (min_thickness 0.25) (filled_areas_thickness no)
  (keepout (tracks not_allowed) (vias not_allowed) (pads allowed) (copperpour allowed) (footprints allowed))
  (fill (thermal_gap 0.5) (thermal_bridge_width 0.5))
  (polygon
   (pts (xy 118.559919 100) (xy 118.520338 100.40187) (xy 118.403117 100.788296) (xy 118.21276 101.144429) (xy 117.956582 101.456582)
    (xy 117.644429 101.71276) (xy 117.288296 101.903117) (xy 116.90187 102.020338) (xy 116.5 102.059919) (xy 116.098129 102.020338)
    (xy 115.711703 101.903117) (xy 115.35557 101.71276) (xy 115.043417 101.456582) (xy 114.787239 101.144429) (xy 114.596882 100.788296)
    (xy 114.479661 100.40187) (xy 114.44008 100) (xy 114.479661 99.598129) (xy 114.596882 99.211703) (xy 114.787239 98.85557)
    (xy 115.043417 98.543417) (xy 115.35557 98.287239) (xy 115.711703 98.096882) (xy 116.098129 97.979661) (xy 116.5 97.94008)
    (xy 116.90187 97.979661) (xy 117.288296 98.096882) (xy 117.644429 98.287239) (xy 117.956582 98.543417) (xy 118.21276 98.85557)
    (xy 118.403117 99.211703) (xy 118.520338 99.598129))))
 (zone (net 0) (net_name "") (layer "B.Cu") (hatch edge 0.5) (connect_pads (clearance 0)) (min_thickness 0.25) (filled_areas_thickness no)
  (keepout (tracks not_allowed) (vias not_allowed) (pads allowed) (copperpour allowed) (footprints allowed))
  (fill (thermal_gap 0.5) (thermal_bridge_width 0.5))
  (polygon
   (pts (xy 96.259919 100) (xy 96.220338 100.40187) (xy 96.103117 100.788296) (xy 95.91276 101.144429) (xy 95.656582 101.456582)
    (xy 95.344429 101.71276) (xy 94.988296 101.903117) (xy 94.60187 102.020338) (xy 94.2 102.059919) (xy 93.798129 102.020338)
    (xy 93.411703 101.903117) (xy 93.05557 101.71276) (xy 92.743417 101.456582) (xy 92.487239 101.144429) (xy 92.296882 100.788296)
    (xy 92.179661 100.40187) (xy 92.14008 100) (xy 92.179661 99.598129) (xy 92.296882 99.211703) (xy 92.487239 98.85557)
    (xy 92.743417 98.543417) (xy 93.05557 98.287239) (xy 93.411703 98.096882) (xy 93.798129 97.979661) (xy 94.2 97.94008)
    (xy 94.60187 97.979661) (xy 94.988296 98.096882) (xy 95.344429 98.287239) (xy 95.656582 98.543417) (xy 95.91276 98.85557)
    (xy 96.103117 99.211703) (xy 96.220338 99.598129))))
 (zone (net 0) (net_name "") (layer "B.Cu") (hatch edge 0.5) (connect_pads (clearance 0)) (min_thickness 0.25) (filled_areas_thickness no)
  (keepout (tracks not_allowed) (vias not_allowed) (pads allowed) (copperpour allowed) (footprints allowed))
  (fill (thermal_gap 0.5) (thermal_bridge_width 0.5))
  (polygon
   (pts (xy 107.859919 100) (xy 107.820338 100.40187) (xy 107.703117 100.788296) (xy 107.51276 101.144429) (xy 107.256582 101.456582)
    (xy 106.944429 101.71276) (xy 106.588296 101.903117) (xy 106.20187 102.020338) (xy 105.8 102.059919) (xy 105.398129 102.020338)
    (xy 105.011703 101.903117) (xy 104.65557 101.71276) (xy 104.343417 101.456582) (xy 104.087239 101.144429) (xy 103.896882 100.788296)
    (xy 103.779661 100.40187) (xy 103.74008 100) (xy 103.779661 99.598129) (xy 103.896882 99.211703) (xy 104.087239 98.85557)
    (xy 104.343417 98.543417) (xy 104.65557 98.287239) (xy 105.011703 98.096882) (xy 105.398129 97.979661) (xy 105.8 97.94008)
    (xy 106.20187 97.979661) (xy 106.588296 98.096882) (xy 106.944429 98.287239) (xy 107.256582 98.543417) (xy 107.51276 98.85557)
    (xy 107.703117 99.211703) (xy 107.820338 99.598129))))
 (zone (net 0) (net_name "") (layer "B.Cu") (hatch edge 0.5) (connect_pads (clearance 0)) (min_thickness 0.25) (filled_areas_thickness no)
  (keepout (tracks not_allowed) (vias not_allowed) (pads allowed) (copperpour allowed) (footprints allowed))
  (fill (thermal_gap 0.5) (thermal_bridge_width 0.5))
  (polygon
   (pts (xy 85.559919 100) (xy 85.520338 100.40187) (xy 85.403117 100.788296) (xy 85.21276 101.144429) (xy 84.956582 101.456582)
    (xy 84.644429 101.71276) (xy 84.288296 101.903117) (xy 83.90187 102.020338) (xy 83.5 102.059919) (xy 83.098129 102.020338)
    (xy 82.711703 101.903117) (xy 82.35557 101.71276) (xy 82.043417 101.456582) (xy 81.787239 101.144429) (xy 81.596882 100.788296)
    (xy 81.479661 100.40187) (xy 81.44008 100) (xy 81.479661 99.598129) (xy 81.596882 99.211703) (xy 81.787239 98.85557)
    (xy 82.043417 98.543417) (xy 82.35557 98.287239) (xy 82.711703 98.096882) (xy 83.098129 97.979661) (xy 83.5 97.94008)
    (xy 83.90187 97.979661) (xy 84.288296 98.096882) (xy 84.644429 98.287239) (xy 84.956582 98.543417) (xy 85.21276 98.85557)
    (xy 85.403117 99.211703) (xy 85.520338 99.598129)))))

